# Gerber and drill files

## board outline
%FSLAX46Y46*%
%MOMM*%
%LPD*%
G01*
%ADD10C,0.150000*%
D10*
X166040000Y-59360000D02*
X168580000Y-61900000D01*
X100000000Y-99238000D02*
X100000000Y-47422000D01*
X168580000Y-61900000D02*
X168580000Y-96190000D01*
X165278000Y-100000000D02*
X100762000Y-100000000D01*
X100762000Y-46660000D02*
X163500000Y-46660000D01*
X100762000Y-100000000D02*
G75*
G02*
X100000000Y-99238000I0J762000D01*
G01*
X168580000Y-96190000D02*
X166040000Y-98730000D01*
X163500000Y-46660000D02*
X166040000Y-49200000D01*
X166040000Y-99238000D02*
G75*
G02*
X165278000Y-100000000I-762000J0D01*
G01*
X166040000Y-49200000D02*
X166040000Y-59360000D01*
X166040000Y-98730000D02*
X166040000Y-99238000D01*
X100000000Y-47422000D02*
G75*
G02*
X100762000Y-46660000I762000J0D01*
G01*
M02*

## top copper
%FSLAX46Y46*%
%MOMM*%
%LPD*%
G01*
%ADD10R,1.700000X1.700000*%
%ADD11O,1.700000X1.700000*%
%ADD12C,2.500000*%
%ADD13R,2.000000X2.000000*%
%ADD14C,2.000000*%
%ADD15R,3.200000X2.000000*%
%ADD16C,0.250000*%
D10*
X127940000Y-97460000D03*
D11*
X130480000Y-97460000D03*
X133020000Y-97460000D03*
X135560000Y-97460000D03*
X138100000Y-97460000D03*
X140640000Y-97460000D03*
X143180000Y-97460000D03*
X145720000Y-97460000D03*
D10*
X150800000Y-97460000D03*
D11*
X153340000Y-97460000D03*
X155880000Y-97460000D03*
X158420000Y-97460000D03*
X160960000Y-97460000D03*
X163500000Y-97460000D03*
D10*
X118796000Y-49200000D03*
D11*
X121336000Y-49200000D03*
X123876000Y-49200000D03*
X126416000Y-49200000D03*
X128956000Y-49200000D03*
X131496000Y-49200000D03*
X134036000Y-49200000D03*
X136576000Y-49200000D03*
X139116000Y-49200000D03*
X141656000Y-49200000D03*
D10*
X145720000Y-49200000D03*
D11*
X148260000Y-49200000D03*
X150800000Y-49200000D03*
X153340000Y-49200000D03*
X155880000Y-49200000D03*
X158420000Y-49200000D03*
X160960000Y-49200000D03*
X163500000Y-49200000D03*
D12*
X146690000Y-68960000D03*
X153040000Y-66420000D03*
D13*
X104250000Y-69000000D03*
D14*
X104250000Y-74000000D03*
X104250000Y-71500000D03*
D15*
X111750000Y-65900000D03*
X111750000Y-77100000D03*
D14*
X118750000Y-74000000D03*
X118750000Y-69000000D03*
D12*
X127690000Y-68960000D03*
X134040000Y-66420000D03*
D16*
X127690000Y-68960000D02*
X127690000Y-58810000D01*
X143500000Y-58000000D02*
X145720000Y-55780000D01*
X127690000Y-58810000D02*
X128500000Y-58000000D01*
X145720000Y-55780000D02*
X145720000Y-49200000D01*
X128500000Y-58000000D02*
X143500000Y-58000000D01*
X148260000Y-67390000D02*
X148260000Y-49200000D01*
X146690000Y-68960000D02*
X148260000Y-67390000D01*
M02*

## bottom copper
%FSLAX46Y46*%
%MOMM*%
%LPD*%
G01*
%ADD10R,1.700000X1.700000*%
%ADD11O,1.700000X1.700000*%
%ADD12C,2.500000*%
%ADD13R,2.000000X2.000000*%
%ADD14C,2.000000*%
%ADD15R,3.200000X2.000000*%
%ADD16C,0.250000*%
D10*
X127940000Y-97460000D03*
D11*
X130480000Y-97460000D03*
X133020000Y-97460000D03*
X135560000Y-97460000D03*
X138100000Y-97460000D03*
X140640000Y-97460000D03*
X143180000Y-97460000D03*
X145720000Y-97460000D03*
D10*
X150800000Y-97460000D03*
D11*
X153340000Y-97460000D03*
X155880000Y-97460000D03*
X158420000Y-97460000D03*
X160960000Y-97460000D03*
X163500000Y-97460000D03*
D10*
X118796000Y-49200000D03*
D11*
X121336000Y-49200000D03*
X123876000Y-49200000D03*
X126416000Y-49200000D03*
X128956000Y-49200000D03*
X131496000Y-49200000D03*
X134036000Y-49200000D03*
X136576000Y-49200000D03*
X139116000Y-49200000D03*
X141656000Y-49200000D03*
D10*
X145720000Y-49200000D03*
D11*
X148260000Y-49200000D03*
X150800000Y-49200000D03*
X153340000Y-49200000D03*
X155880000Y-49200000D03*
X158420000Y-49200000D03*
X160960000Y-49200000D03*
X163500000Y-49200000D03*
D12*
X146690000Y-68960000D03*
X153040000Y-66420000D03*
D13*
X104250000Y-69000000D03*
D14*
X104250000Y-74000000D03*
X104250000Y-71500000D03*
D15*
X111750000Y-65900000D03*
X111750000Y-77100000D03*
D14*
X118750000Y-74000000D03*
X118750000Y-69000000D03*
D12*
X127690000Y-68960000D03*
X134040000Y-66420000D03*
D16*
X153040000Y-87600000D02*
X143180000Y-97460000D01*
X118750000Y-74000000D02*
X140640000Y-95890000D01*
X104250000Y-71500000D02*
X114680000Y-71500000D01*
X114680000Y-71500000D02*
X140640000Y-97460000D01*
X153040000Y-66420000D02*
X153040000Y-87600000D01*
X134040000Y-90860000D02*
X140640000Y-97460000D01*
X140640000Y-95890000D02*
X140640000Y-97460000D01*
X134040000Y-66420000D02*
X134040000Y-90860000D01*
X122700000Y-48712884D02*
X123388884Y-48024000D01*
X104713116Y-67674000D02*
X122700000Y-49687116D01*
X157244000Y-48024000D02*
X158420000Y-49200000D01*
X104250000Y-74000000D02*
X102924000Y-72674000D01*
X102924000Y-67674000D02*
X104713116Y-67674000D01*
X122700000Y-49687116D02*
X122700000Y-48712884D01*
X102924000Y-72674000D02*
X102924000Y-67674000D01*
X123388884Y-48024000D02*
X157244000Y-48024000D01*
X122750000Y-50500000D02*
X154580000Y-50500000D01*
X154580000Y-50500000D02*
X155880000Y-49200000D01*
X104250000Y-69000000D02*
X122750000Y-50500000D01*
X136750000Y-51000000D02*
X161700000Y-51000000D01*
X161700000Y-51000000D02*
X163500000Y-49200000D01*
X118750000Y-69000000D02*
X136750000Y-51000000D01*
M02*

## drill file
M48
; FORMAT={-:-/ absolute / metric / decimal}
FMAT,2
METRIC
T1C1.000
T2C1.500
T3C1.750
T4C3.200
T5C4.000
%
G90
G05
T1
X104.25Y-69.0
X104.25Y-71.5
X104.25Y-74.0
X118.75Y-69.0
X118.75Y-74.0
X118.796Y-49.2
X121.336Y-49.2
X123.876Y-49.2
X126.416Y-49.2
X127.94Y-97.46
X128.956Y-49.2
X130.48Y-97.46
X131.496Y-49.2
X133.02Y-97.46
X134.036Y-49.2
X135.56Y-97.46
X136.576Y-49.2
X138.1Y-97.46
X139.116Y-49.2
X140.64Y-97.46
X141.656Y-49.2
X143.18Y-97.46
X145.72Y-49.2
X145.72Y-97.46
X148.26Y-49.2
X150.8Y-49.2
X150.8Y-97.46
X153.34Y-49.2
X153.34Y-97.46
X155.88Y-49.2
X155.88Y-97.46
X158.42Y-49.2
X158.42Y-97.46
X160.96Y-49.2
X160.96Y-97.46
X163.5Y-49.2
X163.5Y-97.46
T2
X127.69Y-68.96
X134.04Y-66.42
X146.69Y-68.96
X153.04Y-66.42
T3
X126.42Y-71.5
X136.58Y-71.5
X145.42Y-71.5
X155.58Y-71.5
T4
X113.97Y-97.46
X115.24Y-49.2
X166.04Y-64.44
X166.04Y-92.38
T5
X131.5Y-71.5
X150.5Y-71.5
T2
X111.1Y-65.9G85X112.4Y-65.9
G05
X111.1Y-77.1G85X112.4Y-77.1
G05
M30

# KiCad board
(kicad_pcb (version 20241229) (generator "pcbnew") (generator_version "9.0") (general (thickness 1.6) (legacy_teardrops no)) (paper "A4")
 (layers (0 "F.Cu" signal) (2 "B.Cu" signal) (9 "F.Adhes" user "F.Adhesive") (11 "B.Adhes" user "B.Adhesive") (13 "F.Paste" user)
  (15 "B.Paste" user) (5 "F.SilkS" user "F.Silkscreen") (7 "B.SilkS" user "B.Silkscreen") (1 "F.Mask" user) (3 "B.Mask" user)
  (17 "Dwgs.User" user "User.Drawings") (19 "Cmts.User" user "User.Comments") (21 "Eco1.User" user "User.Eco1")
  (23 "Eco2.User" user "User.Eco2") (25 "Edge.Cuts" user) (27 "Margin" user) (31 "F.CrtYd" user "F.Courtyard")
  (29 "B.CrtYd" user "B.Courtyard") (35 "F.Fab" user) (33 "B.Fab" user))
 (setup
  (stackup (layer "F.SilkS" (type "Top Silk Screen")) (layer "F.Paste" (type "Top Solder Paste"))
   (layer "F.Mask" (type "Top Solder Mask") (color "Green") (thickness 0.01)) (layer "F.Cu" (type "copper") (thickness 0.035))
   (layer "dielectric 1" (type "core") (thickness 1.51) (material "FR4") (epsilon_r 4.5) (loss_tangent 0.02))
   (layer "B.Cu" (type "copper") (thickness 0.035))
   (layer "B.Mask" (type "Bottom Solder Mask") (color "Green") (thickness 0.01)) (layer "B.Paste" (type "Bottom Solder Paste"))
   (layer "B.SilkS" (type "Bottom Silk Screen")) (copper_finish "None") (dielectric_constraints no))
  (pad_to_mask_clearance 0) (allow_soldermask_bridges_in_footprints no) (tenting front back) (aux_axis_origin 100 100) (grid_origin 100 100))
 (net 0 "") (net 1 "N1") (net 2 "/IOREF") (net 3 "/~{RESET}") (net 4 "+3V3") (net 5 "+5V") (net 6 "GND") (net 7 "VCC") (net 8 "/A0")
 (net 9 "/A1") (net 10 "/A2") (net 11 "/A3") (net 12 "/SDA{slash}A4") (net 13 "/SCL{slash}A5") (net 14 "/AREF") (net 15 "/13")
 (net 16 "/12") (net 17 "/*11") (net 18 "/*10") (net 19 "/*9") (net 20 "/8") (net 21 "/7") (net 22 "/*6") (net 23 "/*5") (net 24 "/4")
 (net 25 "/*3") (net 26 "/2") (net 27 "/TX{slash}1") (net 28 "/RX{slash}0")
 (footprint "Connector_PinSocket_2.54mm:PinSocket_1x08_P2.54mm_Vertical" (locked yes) (layer "F.Cu") (at 127.94 97.46 90)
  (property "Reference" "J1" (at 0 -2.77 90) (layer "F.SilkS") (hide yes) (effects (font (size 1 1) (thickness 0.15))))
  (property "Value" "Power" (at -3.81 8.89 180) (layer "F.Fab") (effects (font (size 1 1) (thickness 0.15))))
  (pad "1" thru_hole rect (at 0 0 90) (size 1.7 1.7) (drill 1) (layers "*.Cu" "*.Mask") (remove_unused_layers no) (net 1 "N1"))
  (pad "2" thru_hole oval (at 0 2.54 90) (size 1.7 1.7) (drill 1) (layers "*.Cu" "*.Mask") (remove_unused_layers no) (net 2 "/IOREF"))
  (pad "3" thru_hole oval (at 0 5.08 90) (size 1.7 1.7) (drill 1) (layers "*.Cu" "*.Mask") (remove_unused_layers no) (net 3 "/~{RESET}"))
  (pad "4" thru_hole oval (at 0 7.62 90) (size 1.7 1.7) (drill 1) (layers "*.Cu" "*.Mask") (remove_unused_layers no) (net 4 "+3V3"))
  (pad "5" thru_hole oval (at 0 10.16 90) (size 1.7 1.7) (drill 1) (layers "*.Cu" "*.Mask") (remove_unused_layers no) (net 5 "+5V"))
  (pad "6" thru_hole oval (at 0 12.7 90) (size 1.7 1.7) (drill 1) (layers "*.Cu" "*.Mask") (remove_unused_layers no) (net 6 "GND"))
  (pad "7" thru_hole oval (at 0 15.24 90) (size 1.7 1.7) (drill 1) (layers "*.Cu" "*.Mask") (remove_unused_layers no) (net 6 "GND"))
  (pad "8" thru_hole oval (at 0 17.78 90) (size 1.7 1.7) (drill 1) (layers "*.Cu" "*.Mask") (remove_unused_layers no) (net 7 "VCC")))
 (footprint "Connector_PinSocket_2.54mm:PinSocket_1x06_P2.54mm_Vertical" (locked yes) (layer "F.Cu") (at 150.8 97.46 90)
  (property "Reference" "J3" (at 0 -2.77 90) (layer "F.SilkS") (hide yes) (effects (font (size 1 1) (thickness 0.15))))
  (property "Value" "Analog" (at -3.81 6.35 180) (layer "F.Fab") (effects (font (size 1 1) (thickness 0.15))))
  (pad "1" thru_hole rect (at 0 0 90) (size 1.7 1.7) (drill 1) (layers "*.Cu" "*.Mask") (remove_unused_layers no) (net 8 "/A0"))
  (pad "2" thru_hole oval (at 0 2.54 90) (size 1.7 1.7) (drill 1) (layers "*.Cu" "*.Mask") (remove_unused_layers no) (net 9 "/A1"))
  (pad "3" thru_hole oval (at 0 5.08 90) (size 1.7 1.7) (drill 1) (layers "*.Cu" "*.Mask") (remove_unused_layers no) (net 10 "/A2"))
  (pad "4" thru_hole oval (at 0 7.62 90) (size 1.7 1.7) (drill 1) (layers "*.Cu" "*.Mask") (remove_unused_layers no) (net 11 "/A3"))
  (pad "5" thru_hole oval (at 0 10.16 90) (size 1.7 1.7) (drill 1) (layers "*.Cu" "*.Mask") (remove_unused_layers no)
   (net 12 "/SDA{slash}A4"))
  (pad "6" thru_hole oval (at 0 12.7 90) (size 1.7 1.7) (drill 1) (layers "*.Cu" "*.Mask") (remove_unused_layers no)
   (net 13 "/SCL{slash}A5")))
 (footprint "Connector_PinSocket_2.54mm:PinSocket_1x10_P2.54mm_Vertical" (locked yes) (layer "F.Cu") (at 118.796 49.2 90)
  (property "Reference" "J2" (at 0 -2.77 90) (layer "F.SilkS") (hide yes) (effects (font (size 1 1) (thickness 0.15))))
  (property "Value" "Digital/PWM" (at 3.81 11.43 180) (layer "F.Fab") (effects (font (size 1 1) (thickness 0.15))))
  (pad "1" thru_hole rect (at 0 0 90) (size 1.7 1.7) (drill 1) (layers "*.Cu" "*.Mask") (remove_unused_layers no) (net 13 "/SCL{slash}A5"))
  (pad "2" thru_hole oval (at 0 2.54 90) (size 1.7 1.7) (drill 1) (layers "*.Cu" "*.Mask") (remove_unused_layers no)
   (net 12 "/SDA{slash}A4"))
  (pad "3" thru_hole oval (at 0 5.08 90) (size 1.7 1.7) (drill 1) (layers "*.Cu" "*.Mask") (remove_unused_layers no) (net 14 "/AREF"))
  (pad "4" thru_hole oval (at 0 7.62 90) (size 1.7 1.7) (drill 1) (layers "*.Cu" "*.Mask") (remove_unused_layers no) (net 6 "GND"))
  (pad "5" thru_hole oval (at 0 10.16 90) (size 1.7 1.7) (drill 1) (layers "*.Cu" "*.Mask") (remove_unused_layers no) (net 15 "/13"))
  (pad "6" thru_hole oval (at 0 12.7 90) (size 1.7 1.7) (drill 1) (layers "*.Cu" "*.Mask") (remove_unused_layers no) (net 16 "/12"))
  (pad "7" thru_hole oval (at 0 15.24 90) (size 1.7 1.7) (drill 1) (layers "*.Cu" "*.Mask") (remove_unused_layers no) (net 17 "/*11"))
  (pad "8" thru_hole oval (at 0 17.78 90) (size 1.7 1.7) (drill 1) (layers "*.Cu" "*.Mask") (remove_unused_layers no) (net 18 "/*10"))
  (pad "9" thru_hole oval (at 0 20.32 90) (size 1.7 1.7) (drill 1) (layers "*.Cu" "*.Mask") (remove_unused_layers no) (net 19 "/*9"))
  (pad "10" thru_hole oval (at 0 22.86 90) (size 1.7 1.7) (drill 1) (layers "*.Cu" "*.Mask") (remove_unused_layers no) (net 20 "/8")))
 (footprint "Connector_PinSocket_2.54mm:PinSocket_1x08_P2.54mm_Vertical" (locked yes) (layer "F.Cu") (at 145.72 49.2 90)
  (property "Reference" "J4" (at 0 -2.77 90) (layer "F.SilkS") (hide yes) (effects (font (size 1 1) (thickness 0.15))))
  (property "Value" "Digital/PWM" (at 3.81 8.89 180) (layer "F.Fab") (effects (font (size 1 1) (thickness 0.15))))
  (pad "1" thru_hole rect (at 0 0 90) (size 1.7 1.7) (drill 1) (layers "*.Cu" "*.Mask") (remove_unused_layers no) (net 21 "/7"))
  (pad "2" thru_hole oval (at 0 2.54 90) (size 1.7 1.7) (drill 1) (layers "*.Cu" "*.Mask") (remove_unused_layers no) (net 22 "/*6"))
  (pad "3" thru_hole oval (at 0 5.08 90) (size 1.7 1.7) (drill 1) (layers "*.Cu" "*.Mask") (remove_unused_layers no) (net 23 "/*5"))
  (pad "4" thru_hole oval (at 0 7.62 90) (size 1.7 1.7) (drill 1) (layers "*.Cu" "*.Mask") (remove_unused_layers no) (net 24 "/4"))
  (pad "5" thru_hole oval (at 0 10.16 90) (size 1.7 1.7) (drill 1) (layers "*.Cu" "*.Mask") (remove_unused_layers no) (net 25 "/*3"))
  (pad "6" thru_hole oval (at 0 12.7 90) (size 1.7 1.7) (drill 1) (layers "*.Cu" "*.Mask") (remove_unused_layers no) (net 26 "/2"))
  (pad "7" thru_hole oval (at 0 15.24 90) (size 1.7 1.7) (drill 1) (layers "*.Cu" "*.Mask") (remove_unused_layers no) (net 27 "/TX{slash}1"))
  (pad "8" thru_hole oval (at 0 17.78 90) (size 1.7 1.7) (drill 1) (layers "*.Cu" "*.Mask") (remove_unused_layers no) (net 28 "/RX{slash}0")))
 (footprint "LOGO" (layer "F.Cu") (at 112 88.5)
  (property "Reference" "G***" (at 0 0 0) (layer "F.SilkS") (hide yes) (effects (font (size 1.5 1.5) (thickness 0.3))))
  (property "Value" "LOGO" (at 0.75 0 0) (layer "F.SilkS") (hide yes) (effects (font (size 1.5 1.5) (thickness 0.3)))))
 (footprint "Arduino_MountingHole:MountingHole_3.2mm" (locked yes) (layer "F.Cu") (at 115.24 49.2)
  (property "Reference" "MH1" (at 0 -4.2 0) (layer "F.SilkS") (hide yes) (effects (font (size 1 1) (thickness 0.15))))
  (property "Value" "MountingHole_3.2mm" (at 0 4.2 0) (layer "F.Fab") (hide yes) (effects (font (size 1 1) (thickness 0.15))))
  (pad "" np_thru_hole circle (at 0 0) (size 3.2 3.2) (drill 3.2) (layers "*.Cu" "*.Mask")))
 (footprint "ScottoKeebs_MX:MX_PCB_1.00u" (layer "F.Cu") (at 150.5 71.5)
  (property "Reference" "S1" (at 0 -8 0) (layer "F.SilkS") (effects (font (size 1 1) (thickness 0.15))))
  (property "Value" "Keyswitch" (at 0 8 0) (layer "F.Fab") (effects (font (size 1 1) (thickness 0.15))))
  (pad "" np_thru_hole circle (at -5.08 0) (size 1.75 1.75) (drill 1.75) (layers "*.Cu" "*.Mask"))
  (pad "" np_thru_hole circle (at 0 0) (size 4 4) (drill 4) (layers "*.Cu" "*.Mask"))
  (pad "" np_thru_hole circle (at 5.08 0) (size 1.75 1.75) (drill 1.75) (layers "*.Cu" "*.Mask"))
  (pad "1" thru_hole circle (at -3.81 -2.54) (size 2.5 2.5) (drill 1.5) (layers "*.Cu" "*.Mask") (remove_unused_layers no) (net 22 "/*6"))
  (pad "2" thru_hole circle (at 2.54 -5.08) (size 2.5 2.5) (drill 1.5) (layers "*.Cu" "*.Mask") (remove_unused_layers no) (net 6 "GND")))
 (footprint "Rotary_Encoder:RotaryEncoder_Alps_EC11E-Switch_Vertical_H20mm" (layer "F.Cu") (at 104.25 69)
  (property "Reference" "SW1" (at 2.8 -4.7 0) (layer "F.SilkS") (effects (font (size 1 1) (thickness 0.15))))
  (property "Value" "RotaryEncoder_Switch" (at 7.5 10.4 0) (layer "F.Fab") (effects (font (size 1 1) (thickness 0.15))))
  (pad "A" thru_hole rect (at 0 0) (size 2 2) (drill 1) (layers "*.Cu" "*.Mask") (remove_unused_layers no) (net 25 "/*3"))
  (pad "B" thru_hole circle (at 0 5) (size 2 2) (drill 1) (layers "*.Cu" "*.Mask") (remove_unused_layers no) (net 26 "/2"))
  (pad "C" thru_hole circle (at 0 2.5) (size 2 2) (drill 1) (layers "*.Cu" "*.Mask") (remove_unused_layers no) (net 6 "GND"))
  (pad "MP" thru_hole rect (at 7.5 -3.1) (size 3.2 2) (drill oval 2.8 1.5) (layers "*.Cu" "*.Mask") (remove_unused_layers no))
  (pad "MP" thru_hole rect (at 7.5 8.1) (size 3.2 2) (drill oval 2.8 1.5) (layers "*.Cu" "*.Mask") (remove_unused_layers no))
  (pad "S1" thru_hole circle (at 14.5 5) (size 2 2) (drill 1) (layers "*.Cu" "*.Mask") (remove_unused_layers no) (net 6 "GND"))
  (pad "S2" thru_hole circle (at 14.5 0) (size 2 2) (drill 1) (layers "*.Cu" "*.Mask") (remove_unused_layers no) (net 28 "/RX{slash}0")))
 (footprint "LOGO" (layer "F.Cu") (at 112 58 180)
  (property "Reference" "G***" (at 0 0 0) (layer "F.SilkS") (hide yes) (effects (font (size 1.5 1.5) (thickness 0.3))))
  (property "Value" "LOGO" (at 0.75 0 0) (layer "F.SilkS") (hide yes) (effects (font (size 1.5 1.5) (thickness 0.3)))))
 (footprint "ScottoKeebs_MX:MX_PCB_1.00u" (layer "F.Cu") (at 131.5 71.5)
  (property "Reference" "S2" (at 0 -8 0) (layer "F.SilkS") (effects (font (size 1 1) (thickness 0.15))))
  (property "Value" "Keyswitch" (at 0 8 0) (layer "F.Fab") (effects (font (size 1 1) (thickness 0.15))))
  (pad "" np_thru_hole circle (at -5.08 0) (size 1.75 1.75) (drill 1.75) (layers "*.Cu" "*.Mask"))
  (pad "" np_thru_hole circle (at 0 0) (size 4 4) (drill 4) (layers "*.Cu" "*.Mask"))
  (pad "" np_thru_hole circle (at 5.08 0) (size 1.75 1.75) (drill 1.75) (layers "*.Cu" "*.Mask"))
  (pad "1" thru_hole circle (at -3.81 -2.54) (size 2.5 2.5) (drill 1.5) (layers "*.Cu" "*.Mask") (remove_unused_layers no) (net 21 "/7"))
  (pad "2" thru_hole circle (at 2.54 -5.08) (size 2.5 2.5) (drill 1.5) (layers "*.Cu" "*.Mask") (remove_unused_layers no) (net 6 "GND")))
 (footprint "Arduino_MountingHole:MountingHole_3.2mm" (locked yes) (layer "F.Cu") (at 113.97 97.46)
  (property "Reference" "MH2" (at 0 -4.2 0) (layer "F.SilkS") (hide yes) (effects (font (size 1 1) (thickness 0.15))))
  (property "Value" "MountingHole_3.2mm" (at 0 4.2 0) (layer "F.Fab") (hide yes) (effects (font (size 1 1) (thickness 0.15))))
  (pad "" np_thru_hole circle (at 0 0) (size 3.2 3.2) (drill 3.2) (layers "*.Cu" "*.Mask")))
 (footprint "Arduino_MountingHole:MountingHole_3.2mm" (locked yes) (layer "F.Cu") (at 166.04 64.44)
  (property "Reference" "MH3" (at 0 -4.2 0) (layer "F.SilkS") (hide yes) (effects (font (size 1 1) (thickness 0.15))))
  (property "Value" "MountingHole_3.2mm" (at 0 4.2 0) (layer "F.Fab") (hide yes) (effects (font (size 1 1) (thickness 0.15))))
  (pad "" np_thru_hole circle (at 0 0) (size 3.2 3.2) (drill 3.2) (layers "*.Cu" "*.Mask")))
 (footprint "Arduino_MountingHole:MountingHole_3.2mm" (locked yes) (layer "F.Cu") (at 166.04 92.38)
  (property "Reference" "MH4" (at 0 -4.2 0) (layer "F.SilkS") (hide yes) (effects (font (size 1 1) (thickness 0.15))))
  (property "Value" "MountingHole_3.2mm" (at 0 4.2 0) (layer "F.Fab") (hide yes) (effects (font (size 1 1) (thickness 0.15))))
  (pad "" np_thru_hole circle (at 0 0) (size 3.2 3.2) (drill 3.2) (layers "*.Cu" "*.Mask")))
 (gr_line (start 166.04 59.36) (end 168.58 61.9) (stroke (width 0.15) (type solid)) (layer "Edge.Cuts"))
 (gr_line (start 100 99.238) (end 100 47.422) (stroke (width 0.15) (type solid)) (layer "Edge.Cuts"))
 (gr_line (start 168.58 61.9) (end 168.58 96.19) (stroke (width 0.15) (type solid)) (layer "Edge.Cuts"))
 (gr_line (start 165.278 100) (end 100.762 100) (stroke (width 0.15) (type solid)) (layer "Edge.Cuts"))
 (gr_line (start 100.762 46.66) (end 163.5 46.66) (stroke (width 0.15) (type solid)) (layer "Edge.Cuts"))
 (gr_arc (start 100.762 100) (mid 100.223185 99.776815) (end 100 99.238) (stroke (width 0.15) (type solid)) (layer "Edge.Cuts"))
 (gr_line (start 168.58 96.19) (end 166.04 98.73) (stroke (width 0.15) (type solid)) (layer "Edge.Cuts"))
 (gr_line (start 163.5 46.66) (end 166.04 49.2) (stroke (width 0.15) (type solid)) (layer "Edge.Cuts"))
 (gr_arc (start 166.04 99.238) (mid 165.816815 99.776815) (end 165.278 100) (stroke (width 0.15) (type solid)) (layer "Edge.Cuts"))
 (gr_line (start 166.04 49.2) (end 166.04 59.36) (stroke (width 0.15) (type solid)) (layer "Edge.Cuts"))
 (gr_line (start 166.04 98.73) (end 166.04 99.238) (stroke (width 0.15) (type solid)) (layer "Edge.Cuts"))
 (gr_arc (start 100 47.422) (mid 100.223185 46.883185) (end 100.762 46.66) (stroke (width 0.15) (type solid)) (layer "Edge.Cuts"))
 (segment (start 153.04 87.6) (end 143.18 97.46) (width 0.25) (layer "B.Cu") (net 6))
 (segment (start 118.75 74) (end 140.64 95.89) (width 0.25) (layer "B.Cu") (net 6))
 (segment (start 104.25 71.5) (end 114.68 71.5) (width 0.25) (layer "B.Cu") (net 6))
 (segment (start 114.68 71.5) (end 140.64 97.46) (width 0.25) (layer "B.Cu") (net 6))
 (segment (start 153.04 66.42) (end 153.04 87.6) (width 0.25) (layer "B.Cu") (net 6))
 (segment (start 134.04 90.86) (end 140.64 97.46) (width 0.25) (layer "B.Cu") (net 6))
 (segment (start 140.64 95.89) (end 140.64 97.46) (width 0.25) (layer "B.Cu") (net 6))
 (segment (start 134.04 66.42) (end 134.04 90.86) (width 0.25) (layer "B.Cu") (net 6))
 (segment (start 127.69 68.96) (end 127.69 58.81) (width 0.25) (layer "F.Cu") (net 21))
 (segment (start 143.5 58) (end 145.72 55.78) (width 0.25) (layer "F.Cu") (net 21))
 (segment (start 127.69 58.81) (end 128.5 58) (width 0.25) (layer "F.Cu") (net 21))
 (segment (start 145.72 55.78) (end 145.72 49.2) (width 0.25) (layer "F.Cu") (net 21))
 (segment (start 128.5 58) (end 143.5 58) (width 0.25) (layer "F.Cu") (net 21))
 (segment (start 122.7 48.712884) (end 123.388884 48.024) (width 0.25) (layer "B.Cu") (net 26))
 (segment (start 104.713116 67.674) (end 122.7 49.687116) (width 0.25) (layer "B.Cu") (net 26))
 (segment (start 157.244 48.024) (end 158.42 49.2) (width 0.25) (layer "B.Cu") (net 26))
 (segment (start 104.25 74) (end 102.924 72.674) (width 0.25) (layer "B.Cu") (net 26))
 (segment (start 102.924 67.674) (end 104.713116 67.674) (width 0.25) (layer "B.Cu") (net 26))
 (segment (start 122.7 49.687116) (end 122.7 48.712884) (width 0.25) (layer "B.Cu") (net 26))
 (segment (start 102.924 72.674) (end 102.924 67.674) (width 0.25) (layer "B.Cu") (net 26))
 (segment (start 123.388884 48.024) (end 157.244 48.024) (width 0.25) (layer "B.Cu") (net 26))
 (segment (start 148.26 67.39) (end 148.26 49.2) (width 0.25) (layer "F.Cu") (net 22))
 (segment (start 146.69 68.96) (end 148.26 67.39) (width 0.25) (layer "F.Cu") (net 22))
 (segment (start 122.75 50.5) (end 154.58 50.5) (width 0.25) (layer "B.Cu") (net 25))
 (segment (start 154.58 50.5) (end 155.88 49.2) (width 0.25) (layer "B.Cu") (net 25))
 (segment (start 104.25 69) (end 122.75 50.5) (width 0.25) (layer "B.Cu") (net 25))
 (segment (start 136.75 51) (end 161.7 51) (width 0.25) (layer "B.Cu") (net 28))
 (segment (start 161.7 51) (end 163.5 49.2) (width 0.25) (layer "B.Cu") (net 28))
 (segment (start 118.75 69) (end 136.75 51) (width 0.25) (layer "B.Cu") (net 28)))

